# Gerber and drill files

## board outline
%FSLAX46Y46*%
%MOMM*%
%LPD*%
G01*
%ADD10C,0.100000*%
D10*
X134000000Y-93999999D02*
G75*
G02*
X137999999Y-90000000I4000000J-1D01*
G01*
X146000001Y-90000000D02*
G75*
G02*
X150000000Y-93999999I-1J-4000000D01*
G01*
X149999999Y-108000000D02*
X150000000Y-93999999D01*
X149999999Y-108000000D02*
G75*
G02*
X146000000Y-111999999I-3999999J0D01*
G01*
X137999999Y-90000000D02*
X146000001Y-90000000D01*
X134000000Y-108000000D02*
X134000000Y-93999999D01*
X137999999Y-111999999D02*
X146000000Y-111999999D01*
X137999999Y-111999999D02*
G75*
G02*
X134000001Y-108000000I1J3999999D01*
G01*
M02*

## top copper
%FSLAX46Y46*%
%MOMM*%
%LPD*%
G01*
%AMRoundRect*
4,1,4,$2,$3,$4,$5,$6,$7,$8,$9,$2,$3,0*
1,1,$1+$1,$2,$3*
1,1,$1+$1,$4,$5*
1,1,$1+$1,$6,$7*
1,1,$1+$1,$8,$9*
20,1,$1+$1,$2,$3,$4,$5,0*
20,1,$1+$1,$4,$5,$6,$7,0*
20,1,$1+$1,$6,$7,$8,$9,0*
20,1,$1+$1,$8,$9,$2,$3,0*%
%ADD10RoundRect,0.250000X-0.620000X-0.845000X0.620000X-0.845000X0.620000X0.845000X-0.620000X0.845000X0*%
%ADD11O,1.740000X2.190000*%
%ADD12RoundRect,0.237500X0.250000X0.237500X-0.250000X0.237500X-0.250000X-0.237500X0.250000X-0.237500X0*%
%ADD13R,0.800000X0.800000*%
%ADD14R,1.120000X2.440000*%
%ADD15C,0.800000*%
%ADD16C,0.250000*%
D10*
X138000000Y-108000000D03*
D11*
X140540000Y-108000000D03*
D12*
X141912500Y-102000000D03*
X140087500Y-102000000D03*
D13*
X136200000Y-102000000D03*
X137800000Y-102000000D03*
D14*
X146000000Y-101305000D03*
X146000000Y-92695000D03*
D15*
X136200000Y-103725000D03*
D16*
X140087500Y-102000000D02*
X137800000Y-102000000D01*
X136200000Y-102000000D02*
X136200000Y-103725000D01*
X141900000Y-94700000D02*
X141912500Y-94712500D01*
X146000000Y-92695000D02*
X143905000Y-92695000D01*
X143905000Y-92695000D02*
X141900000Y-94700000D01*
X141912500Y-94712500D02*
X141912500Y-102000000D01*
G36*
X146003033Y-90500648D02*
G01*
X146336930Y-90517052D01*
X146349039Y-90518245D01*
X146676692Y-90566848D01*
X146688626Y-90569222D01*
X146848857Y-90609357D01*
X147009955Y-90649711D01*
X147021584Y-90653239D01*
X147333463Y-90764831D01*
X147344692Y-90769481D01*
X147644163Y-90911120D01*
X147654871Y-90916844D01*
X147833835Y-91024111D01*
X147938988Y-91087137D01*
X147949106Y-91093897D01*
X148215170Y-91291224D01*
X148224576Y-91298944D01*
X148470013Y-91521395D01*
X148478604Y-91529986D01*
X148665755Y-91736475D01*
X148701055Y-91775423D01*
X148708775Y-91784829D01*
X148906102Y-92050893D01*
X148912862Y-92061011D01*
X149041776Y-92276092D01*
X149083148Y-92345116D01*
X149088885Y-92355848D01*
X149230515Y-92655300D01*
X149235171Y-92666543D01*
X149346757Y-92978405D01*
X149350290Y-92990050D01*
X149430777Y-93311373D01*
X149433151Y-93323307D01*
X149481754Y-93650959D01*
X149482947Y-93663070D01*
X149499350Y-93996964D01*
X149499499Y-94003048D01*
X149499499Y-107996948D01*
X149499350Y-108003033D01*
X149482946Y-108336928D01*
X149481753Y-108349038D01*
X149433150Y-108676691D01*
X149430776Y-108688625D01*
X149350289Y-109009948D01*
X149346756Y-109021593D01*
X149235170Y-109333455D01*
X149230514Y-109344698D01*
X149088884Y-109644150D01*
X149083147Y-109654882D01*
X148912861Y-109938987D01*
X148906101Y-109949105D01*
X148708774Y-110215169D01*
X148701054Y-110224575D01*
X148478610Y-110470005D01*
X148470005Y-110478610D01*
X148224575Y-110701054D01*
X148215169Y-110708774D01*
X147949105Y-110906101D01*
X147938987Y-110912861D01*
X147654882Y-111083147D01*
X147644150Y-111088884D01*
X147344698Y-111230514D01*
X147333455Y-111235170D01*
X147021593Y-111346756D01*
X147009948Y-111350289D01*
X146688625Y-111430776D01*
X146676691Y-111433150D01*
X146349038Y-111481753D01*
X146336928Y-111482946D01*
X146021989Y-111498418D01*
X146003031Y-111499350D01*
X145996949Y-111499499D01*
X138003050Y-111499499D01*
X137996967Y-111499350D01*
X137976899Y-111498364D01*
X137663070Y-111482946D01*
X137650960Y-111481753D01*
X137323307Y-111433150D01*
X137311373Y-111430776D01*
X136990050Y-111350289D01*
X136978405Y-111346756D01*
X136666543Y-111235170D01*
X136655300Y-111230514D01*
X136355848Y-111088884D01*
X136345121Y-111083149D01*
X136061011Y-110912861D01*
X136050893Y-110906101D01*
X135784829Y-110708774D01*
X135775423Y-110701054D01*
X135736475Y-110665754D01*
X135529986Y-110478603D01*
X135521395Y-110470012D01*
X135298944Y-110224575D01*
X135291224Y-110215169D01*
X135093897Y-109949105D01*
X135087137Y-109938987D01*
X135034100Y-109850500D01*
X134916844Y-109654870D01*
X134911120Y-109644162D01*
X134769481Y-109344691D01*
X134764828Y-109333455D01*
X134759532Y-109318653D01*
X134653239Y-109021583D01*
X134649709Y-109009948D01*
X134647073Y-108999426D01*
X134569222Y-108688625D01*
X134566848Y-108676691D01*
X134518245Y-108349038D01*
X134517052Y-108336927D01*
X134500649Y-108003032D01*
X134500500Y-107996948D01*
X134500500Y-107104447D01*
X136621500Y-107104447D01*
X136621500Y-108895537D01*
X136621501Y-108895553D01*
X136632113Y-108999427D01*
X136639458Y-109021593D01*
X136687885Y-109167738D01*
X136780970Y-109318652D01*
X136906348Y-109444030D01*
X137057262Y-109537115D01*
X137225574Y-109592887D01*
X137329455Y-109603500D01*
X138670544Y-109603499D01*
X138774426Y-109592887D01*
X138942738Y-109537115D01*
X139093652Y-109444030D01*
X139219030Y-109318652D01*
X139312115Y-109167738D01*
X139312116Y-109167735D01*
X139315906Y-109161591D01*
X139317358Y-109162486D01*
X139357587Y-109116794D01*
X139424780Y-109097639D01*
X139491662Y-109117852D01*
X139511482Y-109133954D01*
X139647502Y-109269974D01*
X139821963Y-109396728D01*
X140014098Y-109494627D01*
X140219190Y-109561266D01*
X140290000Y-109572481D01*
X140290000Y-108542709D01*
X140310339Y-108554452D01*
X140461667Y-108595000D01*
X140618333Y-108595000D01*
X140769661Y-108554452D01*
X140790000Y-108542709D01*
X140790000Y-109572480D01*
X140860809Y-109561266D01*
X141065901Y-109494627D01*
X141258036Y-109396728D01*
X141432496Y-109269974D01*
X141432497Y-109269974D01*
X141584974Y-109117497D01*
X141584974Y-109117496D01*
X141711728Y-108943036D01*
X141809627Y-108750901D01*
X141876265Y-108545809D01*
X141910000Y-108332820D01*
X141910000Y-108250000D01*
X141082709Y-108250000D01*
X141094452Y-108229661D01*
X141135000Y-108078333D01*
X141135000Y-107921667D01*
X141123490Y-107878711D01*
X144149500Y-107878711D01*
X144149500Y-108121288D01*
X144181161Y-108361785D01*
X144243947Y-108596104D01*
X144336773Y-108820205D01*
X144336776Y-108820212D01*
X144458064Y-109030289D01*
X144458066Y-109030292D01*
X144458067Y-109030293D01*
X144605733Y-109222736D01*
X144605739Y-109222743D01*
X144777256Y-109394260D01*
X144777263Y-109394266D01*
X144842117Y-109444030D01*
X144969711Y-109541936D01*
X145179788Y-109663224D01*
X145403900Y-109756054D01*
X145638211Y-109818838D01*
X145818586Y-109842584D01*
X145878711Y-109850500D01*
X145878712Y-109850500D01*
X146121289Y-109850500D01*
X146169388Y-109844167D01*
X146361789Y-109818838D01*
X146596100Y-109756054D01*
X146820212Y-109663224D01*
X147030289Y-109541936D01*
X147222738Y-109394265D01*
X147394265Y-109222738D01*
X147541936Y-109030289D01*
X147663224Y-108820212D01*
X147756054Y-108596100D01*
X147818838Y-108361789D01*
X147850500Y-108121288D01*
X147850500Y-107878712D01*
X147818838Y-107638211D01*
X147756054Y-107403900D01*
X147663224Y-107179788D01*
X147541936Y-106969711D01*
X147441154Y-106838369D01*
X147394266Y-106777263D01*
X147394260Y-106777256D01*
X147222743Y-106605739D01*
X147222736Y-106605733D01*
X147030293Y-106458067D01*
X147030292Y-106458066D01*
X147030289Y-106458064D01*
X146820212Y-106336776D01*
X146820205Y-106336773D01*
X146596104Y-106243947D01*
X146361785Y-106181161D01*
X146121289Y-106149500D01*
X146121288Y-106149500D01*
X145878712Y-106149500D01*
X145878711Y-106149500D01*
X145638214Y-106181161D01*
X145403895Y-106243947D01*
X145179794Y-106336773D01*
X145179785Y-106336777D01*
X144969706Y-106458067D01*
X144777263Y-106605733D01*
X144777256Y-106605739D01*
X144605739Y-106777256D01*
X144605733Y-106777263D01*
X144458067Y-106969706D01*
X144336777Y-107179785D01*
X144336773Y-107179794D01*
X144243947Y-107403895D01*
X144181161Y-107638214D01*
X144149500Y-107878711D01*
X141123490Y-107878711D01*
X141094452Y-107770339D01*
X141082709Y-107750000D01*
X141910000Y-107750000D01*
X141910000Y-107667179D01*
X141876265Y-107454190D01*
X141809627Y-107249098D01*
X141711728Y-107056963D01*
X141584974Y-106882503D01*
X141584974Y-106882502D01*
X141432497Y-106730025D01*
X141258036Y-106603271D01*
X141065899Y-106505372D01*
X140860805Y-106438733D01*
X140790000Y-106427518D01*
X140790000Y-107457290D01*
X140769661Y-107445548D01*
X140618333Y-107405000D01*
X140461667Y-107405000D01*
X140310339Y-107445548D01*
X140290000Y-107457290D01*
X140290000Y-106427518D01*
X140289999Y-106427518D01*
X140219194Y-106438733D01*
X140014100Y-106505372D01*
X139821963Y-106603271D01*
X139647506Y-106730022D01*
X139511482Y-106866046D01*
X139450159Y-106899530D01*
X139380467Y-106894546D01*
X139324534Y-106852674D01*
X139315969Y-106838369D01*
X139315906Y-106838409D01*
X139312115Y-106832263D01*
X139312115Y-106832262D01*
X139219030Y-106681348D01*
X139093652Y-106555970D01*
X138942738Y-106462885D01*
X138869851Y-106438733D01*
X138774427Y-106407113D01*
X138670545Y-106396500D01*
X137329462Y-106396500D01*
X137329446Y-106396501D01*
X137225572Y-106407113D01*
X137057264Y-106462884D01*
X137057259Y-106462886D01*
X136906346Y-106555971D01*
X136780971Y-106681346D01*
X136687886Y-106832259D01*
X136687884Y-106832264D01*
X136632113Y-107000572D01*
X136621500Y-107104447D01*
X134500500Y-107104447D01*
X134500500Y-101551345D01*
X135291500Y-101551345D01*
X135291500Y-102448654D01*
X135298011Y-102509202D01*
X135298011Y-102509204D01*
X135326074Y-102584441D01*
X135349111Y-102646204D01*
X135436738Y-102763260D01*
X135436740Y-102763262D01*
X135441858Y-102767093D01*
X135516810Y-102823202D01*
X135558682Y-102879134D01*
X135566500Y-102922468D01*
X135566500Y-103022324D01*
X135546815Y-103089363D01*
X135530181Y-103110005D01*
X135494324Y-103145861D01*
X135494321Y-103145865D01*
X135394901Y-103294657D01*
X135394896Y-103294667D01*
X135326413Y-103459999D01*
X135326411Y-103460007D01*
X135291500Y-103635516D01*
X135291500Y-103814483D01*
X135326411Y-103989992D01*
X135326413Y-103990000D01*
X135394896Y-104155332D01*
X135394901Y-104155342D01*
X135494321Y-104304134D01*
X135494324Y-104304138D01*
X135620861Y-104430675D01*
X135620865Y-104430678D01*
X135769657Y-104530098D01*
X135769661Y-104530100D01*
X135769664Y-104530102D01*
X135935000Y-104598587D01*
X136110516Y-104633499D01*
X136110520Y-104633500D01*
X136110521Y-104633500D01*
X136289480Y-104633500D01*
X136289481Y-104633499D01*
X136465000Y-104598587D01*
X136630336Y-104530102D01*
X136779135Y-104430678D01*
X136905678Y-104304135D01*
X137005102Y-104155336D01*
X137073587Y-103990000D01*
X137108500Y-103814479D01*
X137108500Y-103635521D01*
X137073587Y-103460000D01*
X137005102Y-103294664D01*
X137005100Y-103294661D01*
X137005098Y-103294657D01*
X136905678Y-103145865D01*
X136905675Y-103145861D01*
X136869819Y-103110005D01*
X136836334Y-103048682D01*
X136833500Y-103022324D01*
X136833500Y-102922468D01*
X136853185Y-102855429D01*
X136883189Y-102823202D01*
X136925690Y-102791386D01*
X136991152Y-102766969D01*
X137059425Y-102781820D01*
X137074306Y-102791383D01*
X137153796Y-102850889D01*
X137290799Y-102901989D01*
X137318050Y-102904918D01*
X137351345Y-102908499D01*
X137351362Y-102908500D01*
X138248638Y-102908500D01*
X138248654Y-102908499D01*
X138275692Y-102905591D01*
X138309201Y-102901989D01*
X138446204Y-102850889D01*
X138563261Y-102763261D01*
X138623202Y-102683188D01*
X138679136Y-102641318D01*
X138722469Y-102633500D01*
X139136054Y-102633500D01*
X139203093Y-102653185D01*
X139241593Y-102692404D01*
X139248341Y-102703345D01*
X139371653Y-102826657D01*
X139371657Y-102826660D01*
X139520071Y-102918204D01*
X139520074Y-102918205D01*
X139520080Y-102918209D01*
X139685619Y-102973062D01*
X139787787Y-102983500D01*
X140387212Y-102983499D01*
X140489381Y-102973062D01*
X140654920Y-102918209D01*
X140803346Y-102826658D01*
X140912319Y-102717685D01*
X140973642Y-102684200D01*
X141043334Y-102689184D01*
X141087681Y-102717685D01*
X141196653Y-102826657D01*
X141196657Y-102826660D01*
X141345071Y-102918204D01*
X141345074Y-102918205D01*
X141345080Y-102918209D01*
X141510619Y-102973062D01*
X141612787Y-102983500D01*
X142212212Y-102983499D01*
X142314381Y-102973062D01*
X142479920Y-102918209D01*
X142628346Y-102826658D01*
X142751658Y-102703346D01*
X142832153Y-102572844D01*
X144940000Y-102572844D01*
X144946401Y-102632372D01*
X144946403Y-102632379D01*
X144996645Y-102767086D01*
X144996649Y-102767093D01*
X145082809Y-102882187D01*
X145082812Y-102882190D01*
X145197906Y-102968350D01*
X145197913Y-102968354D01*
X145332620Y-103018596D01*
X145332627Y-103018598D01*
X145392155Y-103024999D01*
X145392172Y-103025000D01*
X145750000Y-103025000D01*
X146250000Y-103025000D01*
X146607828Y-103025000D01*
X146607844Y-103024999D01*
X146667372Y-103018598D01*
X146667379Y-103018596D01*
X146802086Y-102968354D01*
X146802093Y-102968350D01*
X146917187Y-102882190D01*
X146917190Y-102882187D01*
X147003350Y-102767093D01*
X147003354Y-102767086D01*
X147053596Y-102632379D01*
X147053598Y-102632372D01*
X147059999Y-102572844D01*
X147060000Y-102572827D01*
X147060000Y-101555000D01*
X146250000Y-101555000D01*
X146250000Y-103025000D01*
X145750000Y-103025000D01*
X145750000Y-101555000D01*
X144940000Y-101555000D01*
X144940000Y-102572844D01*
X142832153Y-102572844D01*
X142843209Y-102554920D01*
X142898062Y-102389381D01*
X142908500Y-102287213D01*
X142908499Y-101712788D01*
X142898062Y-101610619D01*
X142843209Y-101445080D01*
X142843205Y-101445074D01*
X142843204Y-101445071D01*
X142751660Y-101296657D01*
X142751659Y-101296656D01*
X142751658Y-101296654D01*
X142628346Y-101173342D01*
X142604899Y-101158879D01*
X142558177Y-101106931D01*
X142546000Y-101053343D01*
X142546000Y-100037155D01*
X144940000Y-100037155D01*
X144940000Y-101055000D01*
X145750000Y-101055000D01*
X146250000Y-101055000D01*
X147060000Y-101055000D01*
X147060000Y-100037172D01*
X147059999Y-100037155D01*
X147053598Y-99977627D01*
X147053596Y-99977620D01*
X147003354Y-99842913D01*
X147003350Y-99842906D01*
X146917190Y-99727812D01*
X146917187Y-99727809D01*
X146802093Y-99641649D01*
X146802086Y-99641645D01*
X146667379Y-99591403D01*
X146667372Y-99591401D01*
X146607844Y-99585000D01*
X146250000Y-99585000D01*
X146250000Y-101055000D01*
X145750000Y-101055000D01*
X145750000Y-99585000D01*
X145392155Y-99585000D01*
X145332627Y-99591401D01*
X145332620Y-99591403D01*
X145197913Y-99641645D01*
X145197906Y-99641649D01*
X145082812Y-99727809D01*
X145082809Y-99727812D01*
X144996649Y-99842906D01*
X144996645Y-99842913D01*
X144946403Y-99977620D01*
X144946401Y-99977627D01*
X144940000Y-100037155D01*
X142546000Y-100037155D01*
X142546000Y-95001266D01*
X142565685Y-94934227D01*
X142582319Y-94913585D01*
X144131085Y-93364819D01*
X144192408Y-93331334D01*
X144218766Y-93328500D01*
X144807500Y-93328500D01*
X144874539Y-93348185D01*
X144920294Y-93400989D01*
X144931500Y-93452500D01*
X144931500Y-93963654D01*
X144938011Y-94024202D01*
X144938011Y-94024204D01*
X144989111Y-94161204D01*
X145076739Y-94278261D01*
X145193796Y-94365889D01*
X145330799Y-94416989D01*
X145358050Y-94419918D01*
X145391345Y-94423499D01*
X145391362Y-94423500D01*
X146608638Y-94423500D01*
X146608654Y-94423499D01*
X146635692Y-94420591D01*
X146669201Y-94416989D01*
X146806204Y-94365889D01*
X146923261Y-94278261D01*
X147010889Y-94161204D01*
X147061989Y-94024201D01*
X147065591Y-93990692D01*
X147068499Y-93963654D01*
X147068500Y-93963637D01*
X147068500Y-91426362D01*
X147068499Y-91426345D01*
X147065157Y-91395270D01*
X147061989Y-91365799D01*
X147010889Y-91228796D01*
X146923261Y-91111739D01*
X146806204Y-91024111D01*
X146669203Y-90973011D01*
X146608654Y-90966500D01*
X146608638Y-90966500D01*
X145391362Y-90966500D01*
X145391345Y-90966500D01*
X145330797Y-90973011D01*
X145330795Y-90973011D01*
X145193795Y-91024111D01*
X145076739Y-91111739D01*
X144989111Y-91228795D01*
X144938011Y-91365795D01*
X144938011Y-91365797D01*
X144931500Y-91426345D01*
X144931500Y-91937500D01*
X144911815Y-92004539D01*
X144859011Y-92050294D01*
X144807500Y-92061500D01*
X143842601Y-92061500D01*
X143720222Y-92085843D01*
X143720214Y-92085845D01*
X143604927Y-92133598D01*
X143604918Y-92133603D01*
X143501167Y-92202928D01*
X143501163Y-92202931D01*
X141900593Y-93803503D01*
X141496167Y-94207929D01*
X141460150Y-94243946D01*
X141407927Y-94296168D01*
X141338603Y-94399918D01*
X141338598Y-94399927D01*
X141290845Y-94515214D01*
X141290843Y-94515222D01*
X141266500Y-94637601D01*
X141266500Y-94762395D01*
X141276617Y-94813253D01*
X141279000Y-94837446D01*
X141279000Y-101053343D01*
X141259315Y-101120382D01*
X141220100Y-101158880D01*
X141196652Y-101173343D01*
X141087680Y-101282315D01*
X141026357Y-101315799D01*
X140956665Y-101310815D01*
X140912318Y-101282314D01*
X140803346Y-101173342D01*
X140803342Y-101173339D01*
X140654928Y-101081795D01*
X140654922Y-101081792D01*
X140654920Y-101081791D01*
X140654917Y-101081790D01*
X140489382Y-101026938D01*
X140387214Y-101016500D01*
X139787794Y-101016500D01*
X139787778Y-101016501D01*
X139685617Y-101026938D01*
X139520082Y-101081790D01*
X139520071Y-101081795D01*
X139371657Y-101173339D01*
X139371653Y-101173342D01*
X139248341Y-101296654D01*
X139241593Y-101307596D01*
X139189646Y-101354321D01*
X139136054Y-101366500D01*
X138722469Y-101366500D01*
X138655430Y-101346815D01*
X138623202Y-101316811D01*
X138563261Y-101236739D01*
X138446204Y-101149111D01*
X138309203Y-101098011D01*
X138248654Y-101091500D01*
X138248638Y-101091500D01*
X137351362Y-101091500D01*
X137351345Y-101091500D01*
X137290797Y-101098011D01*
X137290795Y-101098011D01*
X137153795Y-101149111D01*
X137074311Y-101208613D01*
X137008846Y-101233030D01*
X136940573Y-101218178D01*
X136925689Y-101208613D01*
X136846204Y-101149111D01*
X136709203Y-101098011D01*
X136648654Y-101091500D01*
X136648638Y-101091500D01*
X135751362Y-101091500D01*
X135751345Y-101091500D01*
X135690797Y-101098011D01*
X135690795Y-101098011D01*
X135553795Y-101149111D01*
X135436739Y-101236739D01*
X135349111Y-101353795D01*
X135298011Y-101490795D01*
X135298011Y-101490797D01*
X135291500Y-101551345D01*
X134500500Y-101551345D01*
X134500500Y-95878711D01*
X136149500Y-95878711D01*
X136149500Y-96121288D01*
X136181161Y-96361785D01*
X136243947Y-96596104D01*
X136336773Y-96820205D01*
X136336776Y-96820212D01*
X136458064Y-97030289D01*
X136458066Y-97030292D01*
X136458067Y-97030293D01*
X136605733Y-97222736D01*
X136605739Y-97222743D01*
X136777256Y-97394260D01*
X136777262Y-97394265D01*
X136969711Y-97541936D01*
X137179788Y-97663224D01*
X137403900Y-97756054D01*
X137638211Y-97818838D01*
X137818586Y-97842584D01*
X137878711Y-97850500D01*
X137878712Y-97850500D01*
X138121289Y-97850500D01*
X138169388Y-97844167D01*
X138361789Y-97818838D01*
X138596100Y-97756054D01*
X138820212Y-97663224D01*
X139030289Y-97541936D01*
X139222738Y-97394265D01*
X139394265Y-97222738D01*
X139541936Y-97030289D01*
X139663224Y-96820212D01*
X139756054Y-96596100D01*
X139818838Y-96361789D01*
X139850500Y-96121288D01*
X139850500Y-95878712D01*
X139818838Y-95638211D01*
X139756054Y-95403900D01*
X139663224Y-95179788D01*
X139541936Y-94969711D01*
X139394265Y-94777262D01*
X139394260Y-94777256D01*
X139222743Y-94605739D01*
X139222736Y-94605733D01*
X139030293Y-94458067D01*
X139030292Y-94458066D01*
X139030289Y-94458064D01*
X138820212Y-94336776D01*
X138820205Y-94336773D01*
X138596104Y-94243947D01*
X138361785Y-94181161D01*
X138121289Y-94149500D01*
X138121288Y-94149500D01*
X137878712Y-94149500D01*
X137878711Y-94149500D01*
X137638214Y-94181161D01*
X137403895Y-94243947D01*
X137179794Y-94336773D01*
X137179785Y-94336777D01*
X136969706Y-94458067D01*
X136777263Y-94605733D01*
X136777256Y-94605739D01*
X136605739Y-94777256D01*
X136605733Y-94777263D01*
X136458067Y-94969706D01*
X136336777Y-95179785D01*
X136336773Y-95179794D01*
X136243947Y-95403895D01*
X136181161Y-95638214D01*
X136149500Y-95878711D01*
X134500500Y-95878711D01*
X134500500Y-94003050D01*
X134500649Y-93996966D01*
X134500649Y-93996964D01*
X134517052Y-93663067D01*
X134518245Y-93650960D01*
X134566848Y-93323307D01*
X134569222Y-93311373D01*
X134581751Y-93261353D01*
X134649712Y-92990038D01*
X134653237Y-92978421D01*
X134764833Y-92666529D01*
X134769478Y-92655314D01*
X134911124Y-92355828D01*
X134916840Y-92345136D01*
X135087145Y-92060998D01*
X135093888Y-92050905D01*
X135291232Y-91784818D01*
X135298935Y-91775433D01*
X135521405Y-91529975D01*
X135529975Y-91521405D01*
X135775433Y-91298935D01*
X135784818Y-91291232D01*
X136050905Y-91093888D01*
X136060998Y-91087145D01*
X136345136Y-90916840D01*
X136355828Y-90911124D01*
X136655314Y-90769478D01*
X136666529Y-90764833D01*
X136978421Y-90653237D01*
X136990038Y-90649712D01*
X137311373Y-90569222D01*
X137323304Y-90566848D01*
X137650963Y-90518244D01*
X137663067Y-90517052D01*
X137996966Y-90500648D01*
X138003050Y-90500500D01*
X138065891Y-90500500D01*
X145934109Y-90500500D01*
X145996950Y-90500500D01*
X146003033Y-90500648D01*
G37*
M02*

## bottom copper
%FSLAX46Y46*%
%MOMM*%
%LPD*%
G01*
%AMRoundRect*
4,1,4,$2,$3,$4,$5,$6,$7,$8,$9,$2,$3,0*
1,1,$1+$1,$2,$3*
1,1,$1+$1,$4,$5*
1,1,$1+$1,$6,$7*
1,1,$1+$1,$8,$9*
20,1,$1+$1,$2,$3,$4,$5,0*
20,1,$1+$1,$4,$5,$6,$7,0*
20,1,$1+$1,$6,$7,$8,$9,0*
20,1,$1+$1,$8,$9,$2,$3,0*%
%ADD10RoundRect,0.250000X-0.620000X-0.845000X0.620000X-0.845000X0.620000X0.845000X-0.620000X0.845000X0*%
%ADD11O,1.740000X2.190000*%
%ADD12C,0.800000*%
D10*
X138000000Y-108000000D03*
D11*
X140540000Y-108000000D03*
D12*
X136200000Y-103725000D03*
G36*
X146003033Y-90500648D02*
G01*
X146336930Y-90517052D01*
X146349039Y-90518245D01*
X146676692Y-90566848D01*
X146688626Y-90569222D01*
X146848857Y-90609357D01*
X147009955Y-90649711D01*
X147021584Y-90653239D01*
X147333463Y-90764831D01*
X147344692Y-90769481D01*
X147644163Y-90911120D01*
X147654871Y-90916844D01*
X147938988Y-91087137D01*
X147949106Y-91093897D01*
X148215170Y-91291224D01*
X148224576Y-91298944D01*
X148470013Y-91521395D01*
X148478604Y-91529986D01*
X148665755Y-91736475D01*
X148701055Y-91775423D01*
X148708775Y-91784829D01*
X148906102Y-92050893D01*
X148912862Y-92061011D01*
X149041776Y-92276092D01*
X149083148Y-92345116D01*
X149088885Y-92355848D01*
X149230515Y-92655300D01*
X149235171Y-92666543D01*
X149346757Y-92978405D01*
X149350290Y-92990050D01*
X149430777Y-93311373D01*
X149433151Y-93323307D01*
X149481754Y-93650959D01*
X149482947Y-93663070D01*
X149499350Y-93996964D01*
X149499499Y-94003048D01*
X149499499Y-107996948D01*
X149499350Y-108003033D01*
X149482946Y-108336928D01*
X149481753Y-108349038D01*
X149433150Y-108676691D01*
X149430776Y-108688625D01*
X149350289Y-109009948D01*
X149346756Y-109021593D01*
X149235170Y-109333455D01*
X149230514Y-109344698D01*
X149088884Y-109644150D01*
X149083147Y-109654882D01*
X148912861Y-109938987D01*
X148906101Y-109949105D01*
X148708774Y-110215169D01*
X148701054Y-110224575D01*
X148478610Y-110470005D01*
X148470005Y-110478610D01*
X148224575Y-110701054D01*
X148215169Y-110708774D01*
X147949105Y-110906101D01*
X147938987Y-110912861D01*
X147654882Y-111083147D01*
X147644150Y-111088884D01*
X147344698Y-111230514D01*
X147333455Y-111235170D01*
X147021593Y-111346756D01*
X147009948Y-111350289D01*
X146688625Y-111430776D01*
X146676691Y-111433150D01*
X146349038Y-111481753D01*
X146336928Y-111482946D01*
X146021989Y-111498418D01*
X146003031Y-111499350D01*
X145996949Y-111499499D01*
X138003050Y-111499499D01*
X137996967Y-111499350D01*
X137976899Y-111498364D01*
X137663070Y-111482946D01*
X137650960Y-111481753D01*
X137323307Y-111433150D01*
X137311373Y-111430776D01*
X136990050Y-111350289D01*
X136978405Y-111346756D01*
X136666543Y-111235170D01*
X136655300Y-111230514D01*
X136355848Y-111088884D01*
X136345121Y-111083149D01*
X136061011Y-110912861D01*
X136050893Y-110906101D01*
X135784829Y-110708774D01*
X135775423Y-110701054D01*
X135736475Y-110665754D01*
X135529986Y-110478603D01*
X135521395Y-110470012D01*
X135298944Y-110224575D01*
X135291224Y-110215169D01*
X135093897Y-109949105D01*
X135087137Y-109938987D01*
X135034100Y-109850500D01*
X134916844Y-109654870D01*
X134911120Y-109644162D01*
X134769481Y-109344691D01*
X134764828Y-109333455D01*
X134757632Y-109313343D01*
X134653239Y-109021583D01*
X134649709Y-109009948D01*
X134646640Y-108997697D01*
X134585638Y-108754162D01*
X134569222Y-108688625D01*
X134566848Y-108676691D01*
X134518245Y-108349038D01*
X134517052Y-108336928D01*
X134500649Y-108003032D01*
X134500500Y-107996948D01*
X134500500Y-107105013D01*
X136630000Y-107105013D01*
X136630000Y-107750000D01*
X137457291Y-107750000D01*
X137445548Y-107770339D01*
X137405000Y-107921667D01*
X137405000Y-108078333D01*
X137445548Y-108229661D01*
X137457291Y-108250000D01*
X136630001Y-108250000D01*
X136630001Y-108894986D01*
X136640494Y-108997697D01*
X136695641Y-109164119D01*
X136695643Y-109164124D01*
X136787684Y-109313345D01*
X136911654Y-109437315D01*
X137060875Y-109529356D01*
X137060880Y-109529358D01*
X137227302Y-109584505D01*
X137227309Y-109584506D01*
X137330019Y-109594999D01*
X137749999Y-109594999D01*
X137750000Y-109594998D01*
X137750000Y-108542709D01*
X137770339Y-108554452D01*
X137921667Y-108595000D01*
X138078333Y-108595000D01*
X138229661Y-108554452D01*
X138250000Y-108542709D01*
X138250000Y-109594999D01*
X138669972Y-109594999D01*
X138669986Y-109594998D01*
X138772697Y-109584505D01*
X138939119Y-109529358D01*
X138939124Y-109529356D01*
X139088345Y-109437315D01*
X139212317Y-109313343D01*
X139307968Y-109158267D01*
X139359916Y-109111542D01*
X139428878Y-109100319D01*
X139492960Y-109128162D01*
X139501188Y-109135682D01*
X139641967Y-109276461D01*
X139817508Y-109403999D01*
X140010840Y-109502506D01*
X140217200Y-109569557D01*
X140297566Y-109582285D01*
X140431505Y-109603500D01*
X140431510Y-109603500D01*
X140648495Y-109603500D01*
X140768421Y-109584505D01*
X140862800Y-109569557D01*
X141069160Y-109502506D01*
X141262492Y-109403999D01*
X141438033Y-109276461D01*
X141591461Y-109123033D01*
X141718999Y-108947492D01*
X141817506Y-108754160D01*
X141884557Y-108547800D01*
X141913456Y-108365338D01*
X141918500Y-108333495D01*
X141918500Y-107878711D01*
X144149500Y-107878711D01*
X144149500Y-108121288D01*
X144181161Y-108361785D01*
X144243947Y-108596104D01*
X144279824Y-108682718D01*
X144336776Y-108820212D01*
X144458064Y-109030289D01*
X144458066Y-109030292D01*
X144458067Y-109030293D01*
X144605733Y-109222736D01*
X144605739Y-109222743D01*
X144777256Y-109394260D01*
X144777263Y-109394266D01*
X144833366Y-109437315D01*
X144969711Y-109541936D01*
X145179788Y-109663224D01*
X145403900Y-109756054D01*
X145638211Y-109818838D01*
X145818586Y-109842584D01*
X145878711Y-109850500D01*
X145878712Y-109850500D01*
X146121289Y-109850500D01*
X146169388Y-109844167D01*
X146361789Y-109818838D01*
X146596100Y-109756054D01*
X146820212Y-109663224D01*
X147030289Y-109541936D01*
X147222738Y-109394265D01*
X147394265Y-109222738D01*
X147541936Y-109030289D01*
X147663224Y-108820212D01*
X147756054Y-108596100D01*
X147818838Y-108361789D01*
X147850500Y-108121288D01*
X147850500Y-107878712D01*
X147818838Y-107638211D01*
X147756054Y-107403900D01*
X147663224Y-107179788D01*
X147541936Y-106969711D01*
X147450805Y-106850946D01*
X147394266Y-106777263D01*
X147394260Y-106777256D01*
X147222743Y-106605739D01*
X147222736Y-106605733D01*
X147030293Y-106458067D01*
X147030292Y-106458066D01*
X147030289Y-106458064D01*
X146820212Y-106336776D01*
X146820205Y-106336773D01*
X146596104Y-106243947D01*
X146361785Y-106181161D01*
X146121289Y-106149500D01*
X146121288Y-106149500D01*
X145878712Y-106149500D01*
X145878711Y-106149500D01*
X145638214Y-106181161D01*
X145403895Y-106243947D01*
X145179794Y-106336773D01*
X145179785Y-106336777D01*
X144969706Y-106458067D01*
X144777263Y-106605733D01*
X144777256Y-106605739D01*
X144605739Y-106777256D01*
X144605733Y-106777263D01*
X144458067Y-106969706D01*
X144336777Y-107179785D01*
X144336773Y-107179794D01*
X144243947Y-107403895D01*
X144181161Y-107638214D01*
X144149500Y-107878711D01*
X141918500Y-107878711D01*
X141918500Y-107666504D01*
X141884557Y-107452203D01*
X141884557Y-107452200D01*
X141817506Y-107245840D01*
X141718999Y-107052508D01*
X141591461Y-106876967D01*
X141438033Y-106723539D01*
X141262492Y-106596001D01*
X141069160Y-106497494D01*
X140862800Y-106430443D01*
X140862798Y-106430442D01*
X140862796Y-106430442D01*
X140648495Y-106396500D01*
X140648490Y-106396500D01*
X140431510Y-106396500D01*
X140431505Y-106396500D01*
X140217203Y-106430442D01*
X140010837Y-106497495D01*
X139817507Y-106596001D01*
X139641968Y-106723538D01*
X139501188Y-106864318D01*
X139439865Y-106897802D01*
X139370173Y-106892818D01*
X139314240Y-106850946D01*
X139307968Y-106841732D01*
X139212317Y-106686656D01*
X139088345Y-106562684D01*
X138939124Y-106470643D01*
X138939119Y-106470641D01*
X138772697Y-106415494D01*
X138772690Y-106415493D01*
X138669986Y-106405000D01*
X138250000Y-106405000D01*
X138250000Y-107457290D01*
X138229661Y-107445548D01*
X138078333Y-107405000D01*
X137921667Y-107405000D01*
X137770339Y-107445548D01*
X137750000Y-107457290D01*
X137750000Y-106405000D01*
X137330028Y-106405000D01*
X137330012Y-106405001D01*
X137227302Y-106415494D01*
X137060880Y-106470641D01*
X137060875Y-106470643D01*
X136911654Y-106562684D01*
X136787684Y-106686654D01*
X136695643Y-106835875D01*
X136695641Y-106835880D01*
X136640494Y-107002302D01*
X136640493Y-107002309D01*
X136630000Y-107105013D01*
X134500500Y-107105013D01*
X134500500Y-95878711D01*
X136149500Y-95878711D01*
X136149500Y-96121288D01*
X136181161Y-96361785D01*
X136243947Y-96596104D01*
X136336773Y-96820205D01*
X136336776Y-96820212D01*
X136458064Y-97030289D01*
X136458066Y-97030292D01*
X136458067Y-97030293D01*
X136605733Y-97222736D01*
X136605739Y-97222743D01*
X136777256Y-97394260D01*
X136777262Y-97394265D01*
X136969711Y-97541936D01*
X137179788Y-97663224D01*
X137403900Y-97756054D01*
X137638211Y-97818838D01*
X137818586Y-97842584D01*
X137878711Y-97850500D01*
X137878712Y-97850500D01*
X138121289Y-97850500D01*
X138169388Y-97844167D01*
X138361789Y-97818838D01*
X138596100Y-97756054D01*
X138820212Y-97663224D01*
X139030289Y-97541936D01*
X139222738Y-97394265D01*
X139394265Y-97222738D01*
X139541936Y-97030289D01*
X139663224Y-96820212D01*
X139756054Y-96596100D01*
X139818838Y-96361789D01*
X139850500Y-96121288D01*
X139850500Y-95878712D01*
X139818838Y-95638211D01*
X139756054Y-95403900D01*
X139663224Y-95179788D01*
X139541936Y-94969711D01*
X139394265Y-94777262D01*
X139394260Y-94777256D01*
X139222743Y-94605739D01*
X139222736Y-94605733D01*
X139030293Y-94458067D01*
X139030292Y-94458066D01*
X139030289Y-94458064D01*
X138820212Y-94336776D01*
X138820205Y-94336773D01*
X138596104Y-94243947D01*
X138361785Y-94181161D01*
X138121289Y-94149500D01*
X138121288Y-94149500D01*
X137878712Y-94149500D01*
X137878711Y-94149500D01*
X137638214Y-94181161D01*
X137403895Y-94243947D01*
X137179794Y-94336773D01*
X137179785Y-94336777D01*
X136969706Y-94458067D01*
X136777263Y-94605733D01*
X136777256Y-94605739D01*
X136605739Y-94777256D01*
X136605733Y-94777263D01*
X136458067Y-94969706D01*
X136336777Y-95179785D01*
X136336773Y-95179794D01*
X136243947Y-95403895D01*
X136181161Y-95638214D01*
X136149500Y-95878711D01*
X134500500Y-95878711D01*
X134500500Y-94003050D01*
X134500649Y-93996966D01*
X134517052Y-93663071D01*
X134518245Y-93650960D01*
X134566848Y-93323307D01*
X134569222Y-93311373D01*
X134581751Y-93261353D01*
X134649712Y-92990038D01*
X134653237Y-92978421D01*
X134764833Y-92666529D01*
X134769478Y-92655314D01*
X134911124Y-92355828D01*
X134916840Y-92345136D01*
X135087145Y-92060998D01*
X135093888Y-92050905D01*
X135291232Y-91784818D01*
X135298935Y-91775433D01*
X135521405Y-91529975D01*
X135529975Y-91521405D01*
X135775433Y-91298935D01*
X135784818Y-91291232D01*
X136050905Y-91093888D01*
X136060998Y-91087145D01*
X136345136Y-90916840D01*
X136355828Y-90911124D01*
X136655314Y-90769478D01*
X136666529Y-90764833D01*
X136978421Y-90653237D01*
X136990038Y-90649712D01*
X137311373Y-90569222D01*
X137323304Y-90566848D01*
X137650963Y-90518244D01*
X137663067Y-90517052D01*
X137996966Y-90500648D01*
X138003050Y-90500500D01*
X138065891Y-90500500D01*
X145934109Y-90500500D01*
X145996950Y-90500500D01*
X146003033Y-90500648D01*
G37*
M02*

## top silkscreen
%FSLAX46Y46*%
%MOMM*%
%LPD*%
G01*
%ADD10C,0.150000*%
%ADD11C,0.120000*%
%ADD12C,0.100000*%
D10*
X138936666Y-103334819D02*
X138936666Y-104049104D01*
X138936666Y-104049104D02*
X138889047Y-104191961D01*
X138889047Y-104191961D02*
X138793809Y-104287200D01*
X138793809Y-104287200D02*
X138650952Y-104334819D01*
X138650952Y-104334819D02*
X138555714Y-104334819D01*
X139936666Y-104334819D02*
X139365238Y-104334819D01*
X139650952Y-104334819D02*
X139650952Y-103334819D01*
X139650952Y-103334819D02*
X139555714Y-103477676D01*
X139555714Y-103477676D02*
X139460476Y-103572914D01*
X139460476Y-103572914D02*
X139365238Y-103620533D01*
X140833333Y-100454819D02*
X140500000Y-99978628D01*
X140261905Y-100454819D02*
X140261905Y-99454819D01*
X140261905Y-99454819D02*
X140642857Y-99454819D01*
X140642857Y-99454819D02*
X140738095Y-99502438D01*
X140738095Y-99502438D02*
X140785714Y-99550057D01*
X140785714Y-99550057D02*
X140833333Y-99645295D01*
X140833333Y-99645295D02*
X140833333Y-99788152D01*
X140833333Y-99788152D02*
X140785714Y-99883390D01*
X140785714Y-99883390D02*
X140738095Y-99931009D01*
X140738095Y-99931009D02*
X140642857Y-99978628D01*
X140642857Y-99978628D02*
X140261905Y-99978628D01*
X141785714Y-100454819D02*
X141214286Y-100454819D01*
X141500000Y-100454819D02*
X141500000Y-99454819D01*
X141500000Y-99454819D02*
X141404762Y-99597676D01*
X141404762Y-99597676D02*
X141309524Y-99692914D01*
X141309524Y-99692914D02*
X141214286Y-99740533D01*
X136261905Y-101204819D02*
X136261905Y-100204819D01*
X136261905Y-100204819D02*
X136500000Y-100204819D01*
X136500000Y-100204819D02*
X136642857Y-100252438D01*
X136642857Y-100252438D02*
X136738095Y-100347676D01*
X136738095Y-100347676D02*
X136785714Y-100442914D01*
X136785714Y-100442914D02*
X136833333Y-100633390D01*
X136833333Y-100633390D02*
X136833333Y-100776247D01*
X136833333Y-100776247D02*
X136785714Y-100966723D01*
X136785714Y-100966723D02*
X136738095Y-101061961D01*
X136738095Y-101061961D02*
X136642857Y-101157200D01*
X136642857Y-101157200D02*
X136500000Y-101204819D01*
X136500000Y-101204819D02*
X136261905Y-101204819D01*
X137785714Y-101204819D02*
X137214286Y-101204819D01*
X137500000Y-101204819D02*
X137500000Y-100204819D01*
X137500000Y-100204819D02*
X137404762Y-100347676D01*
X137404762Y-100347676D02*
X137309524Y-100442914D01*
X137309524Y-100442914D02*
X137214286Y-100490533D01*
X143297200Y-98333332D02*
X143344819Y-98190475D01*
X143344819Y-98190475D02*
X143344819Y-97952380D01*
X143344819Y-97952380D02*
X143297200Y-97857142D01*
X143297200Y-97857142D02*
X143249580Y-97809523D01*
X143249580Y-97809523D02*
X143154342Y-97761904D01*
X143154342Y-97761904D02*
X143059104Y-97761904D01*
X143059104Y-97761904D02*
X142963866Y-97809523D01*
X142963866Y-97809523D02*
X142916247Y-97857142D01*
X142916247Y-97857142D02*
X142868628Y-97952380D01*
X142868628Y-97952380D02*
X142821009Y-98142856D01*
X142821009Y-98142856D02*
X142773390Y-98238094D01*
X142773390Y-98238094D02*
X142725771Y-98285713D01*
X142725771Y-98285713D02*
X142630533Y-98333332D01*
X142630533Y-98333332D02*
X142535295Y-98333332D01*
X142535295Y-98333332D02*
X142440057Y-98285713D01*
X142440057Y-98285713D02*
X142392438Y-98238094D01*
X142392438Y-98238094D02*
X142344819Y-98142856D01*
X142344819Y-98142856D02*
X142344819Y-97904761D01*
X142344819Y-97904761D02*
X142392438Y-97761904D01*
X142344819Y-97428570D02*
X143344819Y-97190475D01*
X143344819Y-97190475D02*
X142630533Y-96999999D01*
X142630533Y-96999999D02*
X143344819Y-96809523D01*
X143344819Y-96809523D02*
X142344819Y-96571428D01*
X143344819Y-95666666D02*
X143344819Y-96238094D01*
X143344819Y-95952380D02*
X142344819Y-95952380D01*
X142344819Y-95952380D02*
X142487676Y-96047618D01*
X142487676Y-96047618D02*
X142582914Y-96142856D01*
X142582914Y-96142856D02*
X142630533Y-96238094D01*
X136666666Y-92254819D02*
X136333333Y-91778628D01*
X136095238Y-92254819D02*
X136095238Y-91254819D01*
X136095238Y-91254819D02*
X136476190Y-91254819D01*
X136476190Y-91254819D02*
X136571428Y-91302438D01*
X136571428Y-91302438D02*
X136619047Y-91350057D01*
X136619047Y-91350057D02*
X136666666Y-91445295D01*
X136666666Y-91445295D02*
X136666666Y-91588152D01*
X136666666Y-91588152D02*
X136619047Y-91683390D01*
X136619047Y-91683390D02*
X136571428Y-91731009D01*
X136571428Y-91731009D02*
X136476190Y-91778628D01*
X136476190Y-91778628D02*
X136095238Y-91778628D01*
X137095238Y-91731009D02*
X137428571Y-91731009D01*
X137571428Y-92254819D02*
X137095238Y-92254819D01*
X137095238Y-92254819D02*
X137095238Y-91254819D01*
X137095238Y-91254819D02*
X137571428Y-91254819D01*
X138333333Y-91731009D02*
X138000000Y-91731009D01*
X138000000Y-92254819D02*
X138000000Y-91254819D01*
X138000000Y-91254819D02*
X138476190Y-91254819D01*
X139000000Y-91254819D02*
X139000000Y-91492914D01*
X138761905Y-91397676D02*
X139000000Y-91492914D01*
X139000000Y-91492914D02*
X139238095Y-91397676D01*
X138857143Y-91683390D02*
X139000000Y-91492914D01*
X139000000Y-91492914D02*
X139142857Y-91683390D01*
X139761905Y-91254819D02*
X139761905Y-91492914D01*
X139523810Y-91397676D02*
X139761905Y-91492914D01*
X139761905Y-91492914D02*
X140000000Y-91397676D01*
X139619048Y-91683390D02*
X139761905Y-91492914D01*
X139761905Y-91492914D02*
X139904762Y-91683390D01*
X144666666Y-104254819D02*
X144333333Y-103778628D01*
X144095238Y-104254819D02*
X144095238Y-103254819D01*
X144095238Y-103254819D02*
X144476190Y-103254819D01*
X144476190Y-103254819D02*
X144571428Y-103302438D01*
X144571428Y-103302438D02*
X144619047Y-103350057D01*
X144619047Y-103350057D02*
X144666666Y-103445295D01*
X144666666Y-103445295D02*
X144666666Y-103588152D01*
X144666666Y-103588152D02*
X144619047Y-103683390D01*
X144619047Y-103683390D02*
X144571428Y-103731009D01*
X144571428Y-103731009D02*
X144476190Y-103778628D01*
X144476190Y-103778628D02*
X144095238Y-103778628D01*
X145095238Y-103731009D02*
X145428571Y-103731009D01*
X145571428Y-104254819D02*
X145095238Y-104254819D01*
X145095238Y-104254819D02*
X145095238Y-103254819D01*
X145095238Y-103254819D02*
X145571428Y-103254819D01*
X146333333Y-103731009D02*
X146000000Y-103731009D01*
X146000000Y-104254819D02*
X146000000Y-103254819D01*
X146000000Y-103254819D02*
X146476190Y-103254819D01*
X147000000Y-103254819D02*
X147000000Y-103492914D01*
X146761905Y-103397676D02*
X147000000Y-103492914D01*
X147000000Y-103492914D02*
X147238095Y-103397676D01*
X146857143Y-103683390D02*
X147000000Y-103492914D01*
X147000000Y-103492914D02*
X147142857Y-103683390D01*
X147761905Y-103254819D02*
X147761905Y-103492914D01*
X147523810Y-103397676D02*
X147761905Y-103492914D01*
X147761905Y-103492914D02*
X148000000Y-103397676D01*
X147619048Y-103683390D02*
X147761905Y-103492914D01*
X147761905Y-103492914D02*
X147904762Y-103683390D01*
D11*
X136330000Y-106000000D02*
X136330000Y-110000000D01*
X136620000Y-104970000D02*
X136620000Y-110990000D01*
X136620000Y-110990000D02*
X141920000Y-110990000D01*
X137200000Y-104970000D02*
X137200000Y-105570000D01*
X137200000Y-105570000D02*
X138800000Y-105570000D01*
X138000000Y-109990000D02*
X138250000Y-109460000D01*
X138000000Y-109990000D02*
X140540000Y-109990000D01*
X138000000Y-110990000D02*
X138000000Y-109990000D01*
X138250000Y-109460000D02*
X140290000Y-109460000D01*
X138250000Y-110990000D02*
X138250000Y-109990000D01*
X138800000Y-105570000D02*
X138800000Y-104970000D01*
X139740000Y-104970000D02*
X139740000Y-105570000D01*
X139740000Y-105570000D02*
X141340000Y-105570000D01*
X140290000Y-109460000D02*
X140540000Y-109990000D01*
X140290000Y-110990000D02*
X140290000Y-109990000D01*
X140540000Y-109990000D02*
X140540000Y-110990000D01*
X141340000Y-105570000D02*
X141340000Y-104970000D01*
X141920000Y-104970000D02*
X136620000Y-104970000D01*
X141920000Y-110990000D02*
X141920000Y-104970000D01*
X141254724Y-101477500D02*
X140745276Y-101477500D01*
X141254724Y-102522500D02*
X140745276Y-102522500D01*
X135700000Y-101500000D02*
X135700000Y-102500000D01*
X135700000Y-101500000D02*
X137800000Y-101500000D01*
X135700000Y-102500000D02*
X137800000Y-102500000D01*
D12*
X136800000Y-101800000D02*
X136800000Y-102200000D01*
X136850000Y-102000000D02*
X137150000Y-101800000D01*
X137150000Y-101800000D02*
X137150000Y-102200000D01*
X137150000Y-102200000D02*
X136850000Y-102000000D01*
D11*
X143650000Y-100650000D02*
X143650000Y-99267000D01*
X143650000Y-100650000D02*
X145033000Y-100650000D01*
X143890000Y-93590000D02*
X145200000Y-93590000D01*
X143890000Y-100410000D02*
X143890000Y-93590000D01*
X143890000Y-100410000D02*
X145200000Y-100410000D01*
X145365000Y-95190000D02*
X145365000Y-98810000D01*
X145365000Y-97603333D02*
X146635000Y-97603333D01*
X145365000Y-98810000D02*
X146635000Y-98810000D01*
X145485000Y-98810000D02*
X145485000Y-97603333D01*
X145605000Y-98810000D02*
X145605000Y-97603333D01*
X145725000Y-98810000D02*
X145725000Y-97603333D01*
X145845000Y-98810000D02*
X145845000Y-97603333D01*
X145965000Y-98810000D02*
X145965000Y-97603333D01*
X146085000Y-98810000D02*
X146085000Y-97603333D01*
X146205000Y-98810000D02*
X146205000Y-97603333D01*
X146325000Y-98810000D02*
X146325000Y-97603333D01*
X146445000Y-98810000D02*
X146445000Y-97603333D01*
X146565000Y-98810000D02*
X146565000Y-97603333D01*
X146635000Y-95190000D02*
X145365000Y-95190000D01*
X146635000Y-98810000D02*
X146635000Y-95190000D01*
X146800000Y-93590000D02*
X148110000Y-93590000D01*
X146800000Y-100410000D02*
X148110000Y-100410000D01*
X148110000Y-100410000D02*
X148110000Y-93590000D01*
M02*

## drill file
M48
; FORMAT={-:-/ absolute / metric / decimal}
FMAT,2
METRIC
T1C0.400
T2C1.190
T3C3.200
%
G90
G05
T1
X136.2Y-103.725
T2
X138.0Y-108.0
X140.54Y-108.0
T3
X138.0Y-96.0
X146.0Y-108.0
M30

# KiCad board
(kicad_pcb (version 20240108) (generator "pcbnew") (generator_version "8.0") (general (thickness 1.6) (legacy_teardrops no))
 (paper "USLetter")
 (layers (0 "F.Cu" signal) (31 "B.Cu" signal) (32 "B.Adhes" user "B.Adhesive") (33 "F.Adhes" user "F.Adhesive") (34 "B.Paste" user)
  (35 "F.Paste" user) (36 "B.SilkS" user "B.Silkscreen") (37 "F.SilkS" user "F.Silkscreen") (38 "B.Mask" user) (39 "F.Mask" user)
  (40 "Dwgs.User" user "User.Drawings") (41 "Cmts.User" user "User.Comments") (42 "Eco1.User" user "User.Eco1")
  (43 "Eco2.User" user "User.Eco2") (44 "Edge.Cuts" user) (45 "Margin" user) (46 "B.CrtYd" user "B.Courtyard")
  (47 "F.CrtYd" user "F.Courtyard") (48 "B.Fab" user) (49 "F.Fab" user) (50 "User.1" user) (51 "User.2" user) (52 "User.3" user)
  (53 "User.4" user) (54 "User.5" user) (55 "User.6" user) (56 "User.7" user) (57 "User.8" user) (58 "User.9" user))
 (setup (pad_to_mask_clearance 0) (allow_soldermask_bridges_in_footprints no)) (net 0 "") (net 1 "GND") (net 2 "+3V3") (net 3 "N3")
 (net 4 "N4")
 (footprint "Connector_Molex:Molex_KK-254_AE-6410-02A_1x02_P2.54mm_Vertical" (layer "F.Cu") (at 138 108)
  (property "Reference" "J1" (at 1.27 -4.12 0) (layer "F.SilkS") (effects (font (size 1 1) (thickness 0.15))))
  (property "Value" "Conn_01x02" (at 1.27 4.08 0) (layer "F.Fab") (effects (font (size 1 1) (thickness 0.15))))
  (fp_line (start -1.67 -2) (end -1.67 2) (stroke (width 0.12) (type solid)) (layer "F.SilkS"))
  (fp_line (start -1.38 -3.03) (end -1.38 2.99) (stroke (width 0.12) (type solid)) (layer "F.SilkS"))
  (fp_line (start -1.38 2.99) (end 3.92 2.99) (stroke (width 0.12) (type solid)) (layer "F.SilkS"))
  (fp_line (start -0.8 -3.03) (end -0.8 -2.43) (stroke (width 0.12) (type solid)) (layer "F.SilkS"))
  (fp_line (start -0.8 -2.43) (end 0.8 -2.43) (stroke (width 0.12) (type solid)) (layer "F.SilkS"))
  (fp_line (start 0 1.99) (end 0.25 1.46) (stroke (width 0.12) (type solid)) (layer "F.SilkS"))
  (fp_line (start 0 1.99) (end 2.54 1.99) (stroke (width 0.12) (type solid)) (layer "F.SilkS"))
  (fp_line (start 0 2.99) (end 0 1.99) (stroke (width 0.12) (type solid)) (layer "F.SilkS"))
  (fp_line (start 0.25 1.46) (end 2.29 1.46) (stroke (width 0.12) (type solid)) (layer "F.SilkS"))
  (fp_line (start 0.25 2.99) (end 0.25 1.99) (stroke (width 0.12) (type solid)) (layer "F.SilkS"))
  (fp_line (start 0.8 -2.43) (end 0.8 -3.03) (stroke (width 0.12) (type solid)) (layer "F.SilkS"))
  (fp_line (start 1.74 -3.03) (end 1.74 -2.43) (stroke (width 0.12) (type solid)) (layer "F.SilkS"))
  (fp_line (start 1.74 -2.43) (end 3.34 -2.43) (stroke (width 0.12) (type solid)) (layer "F.SilkS"))
  (fp_line (start 2.29 1.46) (end 2.54 1.99) (stroke (width 0.12) (type solid)) (layer "F.SilkS"))
  (fp_line (start 2.29 2.99) (end 2.29 1.99) (stroke (width 0.12) (type solid)) (layer "F.SilkS"))
  (fp_line (start 2.54 1.99) (end 2.54 2.99) (stroke (width 0.12) (type solid)) (layer "F.SilkS"))
  (fp_line (start 3.34 -2.43) (end 3.34 -3.03) (stroke (width 0.12) (type solid)) (layer "F.SilkS"))
  (fp_line (start 3.92 -3.03) (end -1.38 -3.03) (stroke (width 0.12) (type solid)) (layer "F.SilkS"))
  (fp_line (start 3.92 2.99) (end 3.92 -3.03) (stroke (width 0.12) (type solid)) (layer "F.SilkS"))
  (pad "1" thru_hole roundrect (at 0 0) (size 1.74 2.19) (drill 1.19) (layers "*.Cu" "*.Mask") (remove_unused_layers no)
   (roundrect_rratio 0.143678) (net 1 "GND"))
  (pad "2" thru_hole oval (at 2.54 0) (size 1.74 2.19) (drill 1.19) (layers "*.Cu" "*.Mask") (remove_unused_layers no) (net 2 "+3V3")))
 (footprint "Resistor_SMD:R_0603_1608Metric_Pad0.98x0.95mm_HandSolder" (layer "F.Cu") (at 141 102 180)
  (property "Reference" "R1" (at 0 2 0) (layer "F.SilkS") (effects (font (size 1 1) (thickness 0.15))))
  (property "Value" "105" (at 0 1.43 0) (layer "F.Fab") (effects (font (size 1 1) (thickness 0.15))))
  (fp_line (start -0.254724 0.5225) (end 0.254724 0.5225) (stroke (width 0.12) (type solid)) (layer "F.SilkS"))
  (fp_line (start -0.254724 -0.5225) (end 0.254724 -0.5225) (stroke (width 0.12) (type solid)) (layer "F.SilkS"))
  (pad "1" smd roundrect (at -0.9125 0 180) (size 0.975 0.95) (layers "F.Cu" "F.Paste" "F.Mask") (roundrect_rratio 0.25) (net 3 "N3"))
  (pad "2" smd roundrect (at 0.9125 0 180) (size 0.975 0.95) (layers "F.Cu" "F.Paste" "F.Mask") (roundrect_rratio 0.25) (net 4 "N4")))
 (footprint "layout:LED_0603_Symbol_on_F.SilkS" (layer "F.Cu") (at 137 102)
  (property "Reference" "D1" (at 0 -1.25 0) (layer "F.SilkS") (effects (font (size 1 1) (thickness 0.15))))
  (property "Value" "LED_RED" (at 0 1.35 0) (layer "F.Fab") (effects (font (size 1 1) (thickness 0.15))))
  (fp_line (start -1.3 -0.5) (end -1.3 0.5) (stroke (width 0.12) (type solid)) (layer "F.SilkS"))
  (fp_line (start -1.3 -0.5) (end 0.8 -0.5) (stroke (width 0.12) (type solid)) (layer "F.SilkS"))
  (fp_line (start -1.3 0.5) (end 0.8 0.5) (stroke (width 0.12) (type solid)) (layer "F.SilkS"))
  (fp_line (start -0.2 -0.2) (end -0.2 0.2) (stroke (width 0.1) (type solid)) (layer "F.SilkS"))
  (fp_line (start -0.15 0) (end 0.15 -0.2) (stroke (width 0.1) (type solid)) (layer "F.SilkS"))
  (fp_line (start 0.15 -0.2) (end 0.15 0.2) (stroke (width 0.1) (type solid)) (layer "F.SilkS"))
  (fp_line (start 0.15 0.2) (end -0.15 0) (stroke (width 0.1) (type solid)) (layer "F.SilkS"))
  (pad "1" smd rect (at -0.8 0 180) (size 0.8 0.8) (layers "F.Cu" "F.Paste" "F.Mask") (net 1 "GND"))
  (pad "2" smd rect (at 0.8 0 180) (size 0.8 0.8) (layers "F.Cu" "F.Paste" "F.Mask") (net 4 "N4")))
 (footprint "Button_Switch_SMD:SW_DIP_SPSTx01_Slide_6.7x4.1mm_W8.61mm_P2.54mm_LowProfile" (layer "F.Cu") (at 146 97 90)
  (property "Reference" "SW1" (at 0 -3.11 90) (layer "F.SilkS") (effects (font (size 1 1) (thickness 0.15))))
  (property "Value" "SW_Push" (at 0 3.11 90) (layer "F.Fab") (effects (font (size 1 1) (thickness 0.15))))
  (fp_line (start -3.65 -2.35) (end -2.267 -2.35) (stroke (width 0.12) (type solid)) (layer "F.SilkS"))
  (fp_line (start -3.65 -2.35) (end -3.65 -0.967) (stroke (width 0.12) (type solid)) (layer "F.SilkS"))
  (fp_line (start 3.41 -2.11) (end 3.41 -0.8) (stroke (width 0.12) (type solid)) (layer "F.SilkS"))
  (fp_line (start -3.41 -2.11) (end 3.41 -2.11) (stroke (width 0.12) (type solid)) (layer "F.SilkS"))
  (fp_line (start -3.41 -2.11) (end -3.41 -0.8) (stroke (width 0.12) (type solid)) (layer "F.SilkS"))
  (fp_line (start 1.81 -0.635) (end -1.81 -0.635) (stroke (width 0.12) (type solid)) (layer "F.SilkS"))
  (fp_line (start -0.603333 -0.635) (end -0.603333 0.635) (stroke (width 0.12) (type solid)) (layer "F.SilkS"))
  (fp_line (start -1.81 -0.635) (end -1.81 0.635) (stroke (width 0.12) (type solid)) (layer "F.SilkS"))
  (fp_line (start -1.81 -0.515) (end -0.603333 -0.515) (stroke (width 0.12) (type solid)) (layer "F.SilkS"))
  (fp_line (start -1.81 -0.395) (end -0.603333 -0.395) (stroke (width 0.12) (type solid)) (layer "F.SilkS"))
  (fp_line (start -1.81 -0.275) (end -0.603333 -0.275) (stroke (width 0.12) (type solid)) (layer "F.SilkS"))
  (fp_line (start -1.81 -0.155) (end -0.603333 -0.155) (stroke (width 0.12) (type solid)) (layer "F.SilkS"))
  (fp_line (start -1.81 -0.035) (end -0.603333 -0.035) (stroke (width 0.12) (type solid)) (layer "F.SilkS"))
  (fp_line (start -1.81 0.085) (end -0.603333 0.085) (stroke (width 0.12) (type solid)) (layer "F.SilkS"))
  (fp_line (start -1.81 0.205) (end -0.603333 0.205) (stroke (width 0.12) (type solid)) (layer "F.SilkS"))
  (fp_line (start -1.81 0.325) (end -0.603333 0.325) (stroke (width 0.12) (type solid)) (layer "F.SilkS"))
  (fp_line (start -1.81 0.445) (end -0.603333 0.445) (stroke (width 0.12) (type solid)) (layer "F.SilkS"))
  (fp_line (start -1.81 0.565) (end -0.603333 0.565) (stroke (width 0.12) (type solid)) (layer "F.SilkS"))
  (fp_line (start 1.81 0.635) (end 1.81 -0.635) (stroke (width 0.12) (type solid)) (layer "F.SilkS"))
  (fp_line (start -1.81 0.635) (end 1.81 0.635) (stroke (width 0.12) (type solid)) (layer "F.SilkS"))
  (fp_line (start 3.41 0.8) (end 3.41 2.11) (stroke (width 0.12) (type solid)) (layer "F.SilkS"))
  (fp_line (start -3.41 0.8) (end -3.41 2.11) (stroke (width 0.12) (type solid)) (layer "F.SilkS"))
  (fp_line (start -3.41 2.11) (end 3.41 2.11) (stroke (width 0.12) (type solid)) (layer "F.SilkS"))
  (pad "1" smd rect (at -4.305 0 90) (size 2.44 1.12) (layers "F.Cu" "F.Paste" "F.Mask") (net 2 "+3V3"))
  (pad "2" smd rect (at 4.305 0 90) (size 2.44 1.12) (layers "F.Cu" "F.Paste" "F.Mask") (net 3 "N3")))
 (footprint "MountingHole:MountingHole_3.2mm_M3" (layer "F.Cu") (at 138 96)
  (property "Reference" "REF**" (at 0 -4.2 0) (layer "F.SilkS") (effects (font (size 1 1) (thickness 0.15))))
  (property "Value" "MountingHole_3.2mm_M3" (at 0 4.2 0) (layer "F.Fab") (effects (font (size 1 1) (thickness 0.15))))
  (pad "" np_thru_hole circle (at 0 0) (size 3.2 3.2) (drill 3.2) (layers "*.Cu" "*.Mask")))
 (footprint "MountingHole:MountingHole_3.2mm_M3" (layer "F.Cu") (at 146 108)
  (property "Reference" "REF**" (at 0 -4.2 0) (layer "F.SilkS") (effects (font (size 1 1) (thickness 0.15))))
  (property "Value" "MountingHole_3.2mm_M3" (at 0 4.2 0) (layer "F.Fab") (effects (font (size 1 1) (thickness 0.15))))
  (pad "" np_thru_hole circle (at 0 0) (size 3.2 3.2) (drill 3.2) (layers "*.Cu" "*.Mask")))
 (gr_arc (start 134 93.999999) (mid 135.171573 91.171573) (end 137.999999 90) (stroke (width 0.1) (type default)) (layer "Edge.Cuts"))
 (gr_arc (start 146.000001 90) (mid 148.828427 91.171573) (end 150 93.999999) (stroke (width 0.1) (type default)) (layer "Edge.Cuts"))
 (gr_line (start 149.999999 108) (end 150 93.999999) (stroke (width 0.1) (type default)) (layer "Edge.Cuts"))
 (gr_arc (start 149.999999 108) (mid 148.828426 110.828426) (end 146 111.999999) (stroke (width 0.1) (type default)) (layer "Edge.Cuts"))
 (gr_line (start 137.999999 90) (end 146.000001 90) (stroke (width 0.1) (type default)) (layer "Edge.Cuts"))
 (gr_line (start 134 108) (end 134 93.999999) (stroke (width 0.1) (type default)) (layer "Edge.Cuts"))
 (gr_line (start 137.999999 111.999999) (end 146 111.999999) (stroke (width 0.1) (type default)) (layer "Edge.Cuts"))
 (gr_arc (start 137.999999 111.999999) (mid 135.171573 110.828426) (end 134 108) (stroke (width 0.1) (type default)) (layer "Edge.Cuts"))
 (segment (start 140.0875 102) (end 137.8 102) (width 0.25) (layer "F.Cu") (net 4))
 (segment (start 136.2 102) (end 136.2 103.725) (width 0.25) (layer "F.Cu") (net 1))
 (via (at 136.2 103.725) (size 0.8) (drill 0.4) (layers "F.Cu" "B.Cu") (free yes) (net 1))
 (segment (start 141.9 94.7) (end 141.9125 94.7125) (width 0.25) (layer "F.Cu") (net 3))
 (segment (start 146 92.695) (end 143.905 92.695) (width 0.25) (layer "F.Cu") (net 3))
 (segment (start 143.905 92.695) (end 141.9 94.7) (width 0.25) (layer "F.Cu") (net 3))
 (segment (start 141.9125 94.7125) (end 141.9125 102) (width 0.25) (layer "F.Cu") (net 3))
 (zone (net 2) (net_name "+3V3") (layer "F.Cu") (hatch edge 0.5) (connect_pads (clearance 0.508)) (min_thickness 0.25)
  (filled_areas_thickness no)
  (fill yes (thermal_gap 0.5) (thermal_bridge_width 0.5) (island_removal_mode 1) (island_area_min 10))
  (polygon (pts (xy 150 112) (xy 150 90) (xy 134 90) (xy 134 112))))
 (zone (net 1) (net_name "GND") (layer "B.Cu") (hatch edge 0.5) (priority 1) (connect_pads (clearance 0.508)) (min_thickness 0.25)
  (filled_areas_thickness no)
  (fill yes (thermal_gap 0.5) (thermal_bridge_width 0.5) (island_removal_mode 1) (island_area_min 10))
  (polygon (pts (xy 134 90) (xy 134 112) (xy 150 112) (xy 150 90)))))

